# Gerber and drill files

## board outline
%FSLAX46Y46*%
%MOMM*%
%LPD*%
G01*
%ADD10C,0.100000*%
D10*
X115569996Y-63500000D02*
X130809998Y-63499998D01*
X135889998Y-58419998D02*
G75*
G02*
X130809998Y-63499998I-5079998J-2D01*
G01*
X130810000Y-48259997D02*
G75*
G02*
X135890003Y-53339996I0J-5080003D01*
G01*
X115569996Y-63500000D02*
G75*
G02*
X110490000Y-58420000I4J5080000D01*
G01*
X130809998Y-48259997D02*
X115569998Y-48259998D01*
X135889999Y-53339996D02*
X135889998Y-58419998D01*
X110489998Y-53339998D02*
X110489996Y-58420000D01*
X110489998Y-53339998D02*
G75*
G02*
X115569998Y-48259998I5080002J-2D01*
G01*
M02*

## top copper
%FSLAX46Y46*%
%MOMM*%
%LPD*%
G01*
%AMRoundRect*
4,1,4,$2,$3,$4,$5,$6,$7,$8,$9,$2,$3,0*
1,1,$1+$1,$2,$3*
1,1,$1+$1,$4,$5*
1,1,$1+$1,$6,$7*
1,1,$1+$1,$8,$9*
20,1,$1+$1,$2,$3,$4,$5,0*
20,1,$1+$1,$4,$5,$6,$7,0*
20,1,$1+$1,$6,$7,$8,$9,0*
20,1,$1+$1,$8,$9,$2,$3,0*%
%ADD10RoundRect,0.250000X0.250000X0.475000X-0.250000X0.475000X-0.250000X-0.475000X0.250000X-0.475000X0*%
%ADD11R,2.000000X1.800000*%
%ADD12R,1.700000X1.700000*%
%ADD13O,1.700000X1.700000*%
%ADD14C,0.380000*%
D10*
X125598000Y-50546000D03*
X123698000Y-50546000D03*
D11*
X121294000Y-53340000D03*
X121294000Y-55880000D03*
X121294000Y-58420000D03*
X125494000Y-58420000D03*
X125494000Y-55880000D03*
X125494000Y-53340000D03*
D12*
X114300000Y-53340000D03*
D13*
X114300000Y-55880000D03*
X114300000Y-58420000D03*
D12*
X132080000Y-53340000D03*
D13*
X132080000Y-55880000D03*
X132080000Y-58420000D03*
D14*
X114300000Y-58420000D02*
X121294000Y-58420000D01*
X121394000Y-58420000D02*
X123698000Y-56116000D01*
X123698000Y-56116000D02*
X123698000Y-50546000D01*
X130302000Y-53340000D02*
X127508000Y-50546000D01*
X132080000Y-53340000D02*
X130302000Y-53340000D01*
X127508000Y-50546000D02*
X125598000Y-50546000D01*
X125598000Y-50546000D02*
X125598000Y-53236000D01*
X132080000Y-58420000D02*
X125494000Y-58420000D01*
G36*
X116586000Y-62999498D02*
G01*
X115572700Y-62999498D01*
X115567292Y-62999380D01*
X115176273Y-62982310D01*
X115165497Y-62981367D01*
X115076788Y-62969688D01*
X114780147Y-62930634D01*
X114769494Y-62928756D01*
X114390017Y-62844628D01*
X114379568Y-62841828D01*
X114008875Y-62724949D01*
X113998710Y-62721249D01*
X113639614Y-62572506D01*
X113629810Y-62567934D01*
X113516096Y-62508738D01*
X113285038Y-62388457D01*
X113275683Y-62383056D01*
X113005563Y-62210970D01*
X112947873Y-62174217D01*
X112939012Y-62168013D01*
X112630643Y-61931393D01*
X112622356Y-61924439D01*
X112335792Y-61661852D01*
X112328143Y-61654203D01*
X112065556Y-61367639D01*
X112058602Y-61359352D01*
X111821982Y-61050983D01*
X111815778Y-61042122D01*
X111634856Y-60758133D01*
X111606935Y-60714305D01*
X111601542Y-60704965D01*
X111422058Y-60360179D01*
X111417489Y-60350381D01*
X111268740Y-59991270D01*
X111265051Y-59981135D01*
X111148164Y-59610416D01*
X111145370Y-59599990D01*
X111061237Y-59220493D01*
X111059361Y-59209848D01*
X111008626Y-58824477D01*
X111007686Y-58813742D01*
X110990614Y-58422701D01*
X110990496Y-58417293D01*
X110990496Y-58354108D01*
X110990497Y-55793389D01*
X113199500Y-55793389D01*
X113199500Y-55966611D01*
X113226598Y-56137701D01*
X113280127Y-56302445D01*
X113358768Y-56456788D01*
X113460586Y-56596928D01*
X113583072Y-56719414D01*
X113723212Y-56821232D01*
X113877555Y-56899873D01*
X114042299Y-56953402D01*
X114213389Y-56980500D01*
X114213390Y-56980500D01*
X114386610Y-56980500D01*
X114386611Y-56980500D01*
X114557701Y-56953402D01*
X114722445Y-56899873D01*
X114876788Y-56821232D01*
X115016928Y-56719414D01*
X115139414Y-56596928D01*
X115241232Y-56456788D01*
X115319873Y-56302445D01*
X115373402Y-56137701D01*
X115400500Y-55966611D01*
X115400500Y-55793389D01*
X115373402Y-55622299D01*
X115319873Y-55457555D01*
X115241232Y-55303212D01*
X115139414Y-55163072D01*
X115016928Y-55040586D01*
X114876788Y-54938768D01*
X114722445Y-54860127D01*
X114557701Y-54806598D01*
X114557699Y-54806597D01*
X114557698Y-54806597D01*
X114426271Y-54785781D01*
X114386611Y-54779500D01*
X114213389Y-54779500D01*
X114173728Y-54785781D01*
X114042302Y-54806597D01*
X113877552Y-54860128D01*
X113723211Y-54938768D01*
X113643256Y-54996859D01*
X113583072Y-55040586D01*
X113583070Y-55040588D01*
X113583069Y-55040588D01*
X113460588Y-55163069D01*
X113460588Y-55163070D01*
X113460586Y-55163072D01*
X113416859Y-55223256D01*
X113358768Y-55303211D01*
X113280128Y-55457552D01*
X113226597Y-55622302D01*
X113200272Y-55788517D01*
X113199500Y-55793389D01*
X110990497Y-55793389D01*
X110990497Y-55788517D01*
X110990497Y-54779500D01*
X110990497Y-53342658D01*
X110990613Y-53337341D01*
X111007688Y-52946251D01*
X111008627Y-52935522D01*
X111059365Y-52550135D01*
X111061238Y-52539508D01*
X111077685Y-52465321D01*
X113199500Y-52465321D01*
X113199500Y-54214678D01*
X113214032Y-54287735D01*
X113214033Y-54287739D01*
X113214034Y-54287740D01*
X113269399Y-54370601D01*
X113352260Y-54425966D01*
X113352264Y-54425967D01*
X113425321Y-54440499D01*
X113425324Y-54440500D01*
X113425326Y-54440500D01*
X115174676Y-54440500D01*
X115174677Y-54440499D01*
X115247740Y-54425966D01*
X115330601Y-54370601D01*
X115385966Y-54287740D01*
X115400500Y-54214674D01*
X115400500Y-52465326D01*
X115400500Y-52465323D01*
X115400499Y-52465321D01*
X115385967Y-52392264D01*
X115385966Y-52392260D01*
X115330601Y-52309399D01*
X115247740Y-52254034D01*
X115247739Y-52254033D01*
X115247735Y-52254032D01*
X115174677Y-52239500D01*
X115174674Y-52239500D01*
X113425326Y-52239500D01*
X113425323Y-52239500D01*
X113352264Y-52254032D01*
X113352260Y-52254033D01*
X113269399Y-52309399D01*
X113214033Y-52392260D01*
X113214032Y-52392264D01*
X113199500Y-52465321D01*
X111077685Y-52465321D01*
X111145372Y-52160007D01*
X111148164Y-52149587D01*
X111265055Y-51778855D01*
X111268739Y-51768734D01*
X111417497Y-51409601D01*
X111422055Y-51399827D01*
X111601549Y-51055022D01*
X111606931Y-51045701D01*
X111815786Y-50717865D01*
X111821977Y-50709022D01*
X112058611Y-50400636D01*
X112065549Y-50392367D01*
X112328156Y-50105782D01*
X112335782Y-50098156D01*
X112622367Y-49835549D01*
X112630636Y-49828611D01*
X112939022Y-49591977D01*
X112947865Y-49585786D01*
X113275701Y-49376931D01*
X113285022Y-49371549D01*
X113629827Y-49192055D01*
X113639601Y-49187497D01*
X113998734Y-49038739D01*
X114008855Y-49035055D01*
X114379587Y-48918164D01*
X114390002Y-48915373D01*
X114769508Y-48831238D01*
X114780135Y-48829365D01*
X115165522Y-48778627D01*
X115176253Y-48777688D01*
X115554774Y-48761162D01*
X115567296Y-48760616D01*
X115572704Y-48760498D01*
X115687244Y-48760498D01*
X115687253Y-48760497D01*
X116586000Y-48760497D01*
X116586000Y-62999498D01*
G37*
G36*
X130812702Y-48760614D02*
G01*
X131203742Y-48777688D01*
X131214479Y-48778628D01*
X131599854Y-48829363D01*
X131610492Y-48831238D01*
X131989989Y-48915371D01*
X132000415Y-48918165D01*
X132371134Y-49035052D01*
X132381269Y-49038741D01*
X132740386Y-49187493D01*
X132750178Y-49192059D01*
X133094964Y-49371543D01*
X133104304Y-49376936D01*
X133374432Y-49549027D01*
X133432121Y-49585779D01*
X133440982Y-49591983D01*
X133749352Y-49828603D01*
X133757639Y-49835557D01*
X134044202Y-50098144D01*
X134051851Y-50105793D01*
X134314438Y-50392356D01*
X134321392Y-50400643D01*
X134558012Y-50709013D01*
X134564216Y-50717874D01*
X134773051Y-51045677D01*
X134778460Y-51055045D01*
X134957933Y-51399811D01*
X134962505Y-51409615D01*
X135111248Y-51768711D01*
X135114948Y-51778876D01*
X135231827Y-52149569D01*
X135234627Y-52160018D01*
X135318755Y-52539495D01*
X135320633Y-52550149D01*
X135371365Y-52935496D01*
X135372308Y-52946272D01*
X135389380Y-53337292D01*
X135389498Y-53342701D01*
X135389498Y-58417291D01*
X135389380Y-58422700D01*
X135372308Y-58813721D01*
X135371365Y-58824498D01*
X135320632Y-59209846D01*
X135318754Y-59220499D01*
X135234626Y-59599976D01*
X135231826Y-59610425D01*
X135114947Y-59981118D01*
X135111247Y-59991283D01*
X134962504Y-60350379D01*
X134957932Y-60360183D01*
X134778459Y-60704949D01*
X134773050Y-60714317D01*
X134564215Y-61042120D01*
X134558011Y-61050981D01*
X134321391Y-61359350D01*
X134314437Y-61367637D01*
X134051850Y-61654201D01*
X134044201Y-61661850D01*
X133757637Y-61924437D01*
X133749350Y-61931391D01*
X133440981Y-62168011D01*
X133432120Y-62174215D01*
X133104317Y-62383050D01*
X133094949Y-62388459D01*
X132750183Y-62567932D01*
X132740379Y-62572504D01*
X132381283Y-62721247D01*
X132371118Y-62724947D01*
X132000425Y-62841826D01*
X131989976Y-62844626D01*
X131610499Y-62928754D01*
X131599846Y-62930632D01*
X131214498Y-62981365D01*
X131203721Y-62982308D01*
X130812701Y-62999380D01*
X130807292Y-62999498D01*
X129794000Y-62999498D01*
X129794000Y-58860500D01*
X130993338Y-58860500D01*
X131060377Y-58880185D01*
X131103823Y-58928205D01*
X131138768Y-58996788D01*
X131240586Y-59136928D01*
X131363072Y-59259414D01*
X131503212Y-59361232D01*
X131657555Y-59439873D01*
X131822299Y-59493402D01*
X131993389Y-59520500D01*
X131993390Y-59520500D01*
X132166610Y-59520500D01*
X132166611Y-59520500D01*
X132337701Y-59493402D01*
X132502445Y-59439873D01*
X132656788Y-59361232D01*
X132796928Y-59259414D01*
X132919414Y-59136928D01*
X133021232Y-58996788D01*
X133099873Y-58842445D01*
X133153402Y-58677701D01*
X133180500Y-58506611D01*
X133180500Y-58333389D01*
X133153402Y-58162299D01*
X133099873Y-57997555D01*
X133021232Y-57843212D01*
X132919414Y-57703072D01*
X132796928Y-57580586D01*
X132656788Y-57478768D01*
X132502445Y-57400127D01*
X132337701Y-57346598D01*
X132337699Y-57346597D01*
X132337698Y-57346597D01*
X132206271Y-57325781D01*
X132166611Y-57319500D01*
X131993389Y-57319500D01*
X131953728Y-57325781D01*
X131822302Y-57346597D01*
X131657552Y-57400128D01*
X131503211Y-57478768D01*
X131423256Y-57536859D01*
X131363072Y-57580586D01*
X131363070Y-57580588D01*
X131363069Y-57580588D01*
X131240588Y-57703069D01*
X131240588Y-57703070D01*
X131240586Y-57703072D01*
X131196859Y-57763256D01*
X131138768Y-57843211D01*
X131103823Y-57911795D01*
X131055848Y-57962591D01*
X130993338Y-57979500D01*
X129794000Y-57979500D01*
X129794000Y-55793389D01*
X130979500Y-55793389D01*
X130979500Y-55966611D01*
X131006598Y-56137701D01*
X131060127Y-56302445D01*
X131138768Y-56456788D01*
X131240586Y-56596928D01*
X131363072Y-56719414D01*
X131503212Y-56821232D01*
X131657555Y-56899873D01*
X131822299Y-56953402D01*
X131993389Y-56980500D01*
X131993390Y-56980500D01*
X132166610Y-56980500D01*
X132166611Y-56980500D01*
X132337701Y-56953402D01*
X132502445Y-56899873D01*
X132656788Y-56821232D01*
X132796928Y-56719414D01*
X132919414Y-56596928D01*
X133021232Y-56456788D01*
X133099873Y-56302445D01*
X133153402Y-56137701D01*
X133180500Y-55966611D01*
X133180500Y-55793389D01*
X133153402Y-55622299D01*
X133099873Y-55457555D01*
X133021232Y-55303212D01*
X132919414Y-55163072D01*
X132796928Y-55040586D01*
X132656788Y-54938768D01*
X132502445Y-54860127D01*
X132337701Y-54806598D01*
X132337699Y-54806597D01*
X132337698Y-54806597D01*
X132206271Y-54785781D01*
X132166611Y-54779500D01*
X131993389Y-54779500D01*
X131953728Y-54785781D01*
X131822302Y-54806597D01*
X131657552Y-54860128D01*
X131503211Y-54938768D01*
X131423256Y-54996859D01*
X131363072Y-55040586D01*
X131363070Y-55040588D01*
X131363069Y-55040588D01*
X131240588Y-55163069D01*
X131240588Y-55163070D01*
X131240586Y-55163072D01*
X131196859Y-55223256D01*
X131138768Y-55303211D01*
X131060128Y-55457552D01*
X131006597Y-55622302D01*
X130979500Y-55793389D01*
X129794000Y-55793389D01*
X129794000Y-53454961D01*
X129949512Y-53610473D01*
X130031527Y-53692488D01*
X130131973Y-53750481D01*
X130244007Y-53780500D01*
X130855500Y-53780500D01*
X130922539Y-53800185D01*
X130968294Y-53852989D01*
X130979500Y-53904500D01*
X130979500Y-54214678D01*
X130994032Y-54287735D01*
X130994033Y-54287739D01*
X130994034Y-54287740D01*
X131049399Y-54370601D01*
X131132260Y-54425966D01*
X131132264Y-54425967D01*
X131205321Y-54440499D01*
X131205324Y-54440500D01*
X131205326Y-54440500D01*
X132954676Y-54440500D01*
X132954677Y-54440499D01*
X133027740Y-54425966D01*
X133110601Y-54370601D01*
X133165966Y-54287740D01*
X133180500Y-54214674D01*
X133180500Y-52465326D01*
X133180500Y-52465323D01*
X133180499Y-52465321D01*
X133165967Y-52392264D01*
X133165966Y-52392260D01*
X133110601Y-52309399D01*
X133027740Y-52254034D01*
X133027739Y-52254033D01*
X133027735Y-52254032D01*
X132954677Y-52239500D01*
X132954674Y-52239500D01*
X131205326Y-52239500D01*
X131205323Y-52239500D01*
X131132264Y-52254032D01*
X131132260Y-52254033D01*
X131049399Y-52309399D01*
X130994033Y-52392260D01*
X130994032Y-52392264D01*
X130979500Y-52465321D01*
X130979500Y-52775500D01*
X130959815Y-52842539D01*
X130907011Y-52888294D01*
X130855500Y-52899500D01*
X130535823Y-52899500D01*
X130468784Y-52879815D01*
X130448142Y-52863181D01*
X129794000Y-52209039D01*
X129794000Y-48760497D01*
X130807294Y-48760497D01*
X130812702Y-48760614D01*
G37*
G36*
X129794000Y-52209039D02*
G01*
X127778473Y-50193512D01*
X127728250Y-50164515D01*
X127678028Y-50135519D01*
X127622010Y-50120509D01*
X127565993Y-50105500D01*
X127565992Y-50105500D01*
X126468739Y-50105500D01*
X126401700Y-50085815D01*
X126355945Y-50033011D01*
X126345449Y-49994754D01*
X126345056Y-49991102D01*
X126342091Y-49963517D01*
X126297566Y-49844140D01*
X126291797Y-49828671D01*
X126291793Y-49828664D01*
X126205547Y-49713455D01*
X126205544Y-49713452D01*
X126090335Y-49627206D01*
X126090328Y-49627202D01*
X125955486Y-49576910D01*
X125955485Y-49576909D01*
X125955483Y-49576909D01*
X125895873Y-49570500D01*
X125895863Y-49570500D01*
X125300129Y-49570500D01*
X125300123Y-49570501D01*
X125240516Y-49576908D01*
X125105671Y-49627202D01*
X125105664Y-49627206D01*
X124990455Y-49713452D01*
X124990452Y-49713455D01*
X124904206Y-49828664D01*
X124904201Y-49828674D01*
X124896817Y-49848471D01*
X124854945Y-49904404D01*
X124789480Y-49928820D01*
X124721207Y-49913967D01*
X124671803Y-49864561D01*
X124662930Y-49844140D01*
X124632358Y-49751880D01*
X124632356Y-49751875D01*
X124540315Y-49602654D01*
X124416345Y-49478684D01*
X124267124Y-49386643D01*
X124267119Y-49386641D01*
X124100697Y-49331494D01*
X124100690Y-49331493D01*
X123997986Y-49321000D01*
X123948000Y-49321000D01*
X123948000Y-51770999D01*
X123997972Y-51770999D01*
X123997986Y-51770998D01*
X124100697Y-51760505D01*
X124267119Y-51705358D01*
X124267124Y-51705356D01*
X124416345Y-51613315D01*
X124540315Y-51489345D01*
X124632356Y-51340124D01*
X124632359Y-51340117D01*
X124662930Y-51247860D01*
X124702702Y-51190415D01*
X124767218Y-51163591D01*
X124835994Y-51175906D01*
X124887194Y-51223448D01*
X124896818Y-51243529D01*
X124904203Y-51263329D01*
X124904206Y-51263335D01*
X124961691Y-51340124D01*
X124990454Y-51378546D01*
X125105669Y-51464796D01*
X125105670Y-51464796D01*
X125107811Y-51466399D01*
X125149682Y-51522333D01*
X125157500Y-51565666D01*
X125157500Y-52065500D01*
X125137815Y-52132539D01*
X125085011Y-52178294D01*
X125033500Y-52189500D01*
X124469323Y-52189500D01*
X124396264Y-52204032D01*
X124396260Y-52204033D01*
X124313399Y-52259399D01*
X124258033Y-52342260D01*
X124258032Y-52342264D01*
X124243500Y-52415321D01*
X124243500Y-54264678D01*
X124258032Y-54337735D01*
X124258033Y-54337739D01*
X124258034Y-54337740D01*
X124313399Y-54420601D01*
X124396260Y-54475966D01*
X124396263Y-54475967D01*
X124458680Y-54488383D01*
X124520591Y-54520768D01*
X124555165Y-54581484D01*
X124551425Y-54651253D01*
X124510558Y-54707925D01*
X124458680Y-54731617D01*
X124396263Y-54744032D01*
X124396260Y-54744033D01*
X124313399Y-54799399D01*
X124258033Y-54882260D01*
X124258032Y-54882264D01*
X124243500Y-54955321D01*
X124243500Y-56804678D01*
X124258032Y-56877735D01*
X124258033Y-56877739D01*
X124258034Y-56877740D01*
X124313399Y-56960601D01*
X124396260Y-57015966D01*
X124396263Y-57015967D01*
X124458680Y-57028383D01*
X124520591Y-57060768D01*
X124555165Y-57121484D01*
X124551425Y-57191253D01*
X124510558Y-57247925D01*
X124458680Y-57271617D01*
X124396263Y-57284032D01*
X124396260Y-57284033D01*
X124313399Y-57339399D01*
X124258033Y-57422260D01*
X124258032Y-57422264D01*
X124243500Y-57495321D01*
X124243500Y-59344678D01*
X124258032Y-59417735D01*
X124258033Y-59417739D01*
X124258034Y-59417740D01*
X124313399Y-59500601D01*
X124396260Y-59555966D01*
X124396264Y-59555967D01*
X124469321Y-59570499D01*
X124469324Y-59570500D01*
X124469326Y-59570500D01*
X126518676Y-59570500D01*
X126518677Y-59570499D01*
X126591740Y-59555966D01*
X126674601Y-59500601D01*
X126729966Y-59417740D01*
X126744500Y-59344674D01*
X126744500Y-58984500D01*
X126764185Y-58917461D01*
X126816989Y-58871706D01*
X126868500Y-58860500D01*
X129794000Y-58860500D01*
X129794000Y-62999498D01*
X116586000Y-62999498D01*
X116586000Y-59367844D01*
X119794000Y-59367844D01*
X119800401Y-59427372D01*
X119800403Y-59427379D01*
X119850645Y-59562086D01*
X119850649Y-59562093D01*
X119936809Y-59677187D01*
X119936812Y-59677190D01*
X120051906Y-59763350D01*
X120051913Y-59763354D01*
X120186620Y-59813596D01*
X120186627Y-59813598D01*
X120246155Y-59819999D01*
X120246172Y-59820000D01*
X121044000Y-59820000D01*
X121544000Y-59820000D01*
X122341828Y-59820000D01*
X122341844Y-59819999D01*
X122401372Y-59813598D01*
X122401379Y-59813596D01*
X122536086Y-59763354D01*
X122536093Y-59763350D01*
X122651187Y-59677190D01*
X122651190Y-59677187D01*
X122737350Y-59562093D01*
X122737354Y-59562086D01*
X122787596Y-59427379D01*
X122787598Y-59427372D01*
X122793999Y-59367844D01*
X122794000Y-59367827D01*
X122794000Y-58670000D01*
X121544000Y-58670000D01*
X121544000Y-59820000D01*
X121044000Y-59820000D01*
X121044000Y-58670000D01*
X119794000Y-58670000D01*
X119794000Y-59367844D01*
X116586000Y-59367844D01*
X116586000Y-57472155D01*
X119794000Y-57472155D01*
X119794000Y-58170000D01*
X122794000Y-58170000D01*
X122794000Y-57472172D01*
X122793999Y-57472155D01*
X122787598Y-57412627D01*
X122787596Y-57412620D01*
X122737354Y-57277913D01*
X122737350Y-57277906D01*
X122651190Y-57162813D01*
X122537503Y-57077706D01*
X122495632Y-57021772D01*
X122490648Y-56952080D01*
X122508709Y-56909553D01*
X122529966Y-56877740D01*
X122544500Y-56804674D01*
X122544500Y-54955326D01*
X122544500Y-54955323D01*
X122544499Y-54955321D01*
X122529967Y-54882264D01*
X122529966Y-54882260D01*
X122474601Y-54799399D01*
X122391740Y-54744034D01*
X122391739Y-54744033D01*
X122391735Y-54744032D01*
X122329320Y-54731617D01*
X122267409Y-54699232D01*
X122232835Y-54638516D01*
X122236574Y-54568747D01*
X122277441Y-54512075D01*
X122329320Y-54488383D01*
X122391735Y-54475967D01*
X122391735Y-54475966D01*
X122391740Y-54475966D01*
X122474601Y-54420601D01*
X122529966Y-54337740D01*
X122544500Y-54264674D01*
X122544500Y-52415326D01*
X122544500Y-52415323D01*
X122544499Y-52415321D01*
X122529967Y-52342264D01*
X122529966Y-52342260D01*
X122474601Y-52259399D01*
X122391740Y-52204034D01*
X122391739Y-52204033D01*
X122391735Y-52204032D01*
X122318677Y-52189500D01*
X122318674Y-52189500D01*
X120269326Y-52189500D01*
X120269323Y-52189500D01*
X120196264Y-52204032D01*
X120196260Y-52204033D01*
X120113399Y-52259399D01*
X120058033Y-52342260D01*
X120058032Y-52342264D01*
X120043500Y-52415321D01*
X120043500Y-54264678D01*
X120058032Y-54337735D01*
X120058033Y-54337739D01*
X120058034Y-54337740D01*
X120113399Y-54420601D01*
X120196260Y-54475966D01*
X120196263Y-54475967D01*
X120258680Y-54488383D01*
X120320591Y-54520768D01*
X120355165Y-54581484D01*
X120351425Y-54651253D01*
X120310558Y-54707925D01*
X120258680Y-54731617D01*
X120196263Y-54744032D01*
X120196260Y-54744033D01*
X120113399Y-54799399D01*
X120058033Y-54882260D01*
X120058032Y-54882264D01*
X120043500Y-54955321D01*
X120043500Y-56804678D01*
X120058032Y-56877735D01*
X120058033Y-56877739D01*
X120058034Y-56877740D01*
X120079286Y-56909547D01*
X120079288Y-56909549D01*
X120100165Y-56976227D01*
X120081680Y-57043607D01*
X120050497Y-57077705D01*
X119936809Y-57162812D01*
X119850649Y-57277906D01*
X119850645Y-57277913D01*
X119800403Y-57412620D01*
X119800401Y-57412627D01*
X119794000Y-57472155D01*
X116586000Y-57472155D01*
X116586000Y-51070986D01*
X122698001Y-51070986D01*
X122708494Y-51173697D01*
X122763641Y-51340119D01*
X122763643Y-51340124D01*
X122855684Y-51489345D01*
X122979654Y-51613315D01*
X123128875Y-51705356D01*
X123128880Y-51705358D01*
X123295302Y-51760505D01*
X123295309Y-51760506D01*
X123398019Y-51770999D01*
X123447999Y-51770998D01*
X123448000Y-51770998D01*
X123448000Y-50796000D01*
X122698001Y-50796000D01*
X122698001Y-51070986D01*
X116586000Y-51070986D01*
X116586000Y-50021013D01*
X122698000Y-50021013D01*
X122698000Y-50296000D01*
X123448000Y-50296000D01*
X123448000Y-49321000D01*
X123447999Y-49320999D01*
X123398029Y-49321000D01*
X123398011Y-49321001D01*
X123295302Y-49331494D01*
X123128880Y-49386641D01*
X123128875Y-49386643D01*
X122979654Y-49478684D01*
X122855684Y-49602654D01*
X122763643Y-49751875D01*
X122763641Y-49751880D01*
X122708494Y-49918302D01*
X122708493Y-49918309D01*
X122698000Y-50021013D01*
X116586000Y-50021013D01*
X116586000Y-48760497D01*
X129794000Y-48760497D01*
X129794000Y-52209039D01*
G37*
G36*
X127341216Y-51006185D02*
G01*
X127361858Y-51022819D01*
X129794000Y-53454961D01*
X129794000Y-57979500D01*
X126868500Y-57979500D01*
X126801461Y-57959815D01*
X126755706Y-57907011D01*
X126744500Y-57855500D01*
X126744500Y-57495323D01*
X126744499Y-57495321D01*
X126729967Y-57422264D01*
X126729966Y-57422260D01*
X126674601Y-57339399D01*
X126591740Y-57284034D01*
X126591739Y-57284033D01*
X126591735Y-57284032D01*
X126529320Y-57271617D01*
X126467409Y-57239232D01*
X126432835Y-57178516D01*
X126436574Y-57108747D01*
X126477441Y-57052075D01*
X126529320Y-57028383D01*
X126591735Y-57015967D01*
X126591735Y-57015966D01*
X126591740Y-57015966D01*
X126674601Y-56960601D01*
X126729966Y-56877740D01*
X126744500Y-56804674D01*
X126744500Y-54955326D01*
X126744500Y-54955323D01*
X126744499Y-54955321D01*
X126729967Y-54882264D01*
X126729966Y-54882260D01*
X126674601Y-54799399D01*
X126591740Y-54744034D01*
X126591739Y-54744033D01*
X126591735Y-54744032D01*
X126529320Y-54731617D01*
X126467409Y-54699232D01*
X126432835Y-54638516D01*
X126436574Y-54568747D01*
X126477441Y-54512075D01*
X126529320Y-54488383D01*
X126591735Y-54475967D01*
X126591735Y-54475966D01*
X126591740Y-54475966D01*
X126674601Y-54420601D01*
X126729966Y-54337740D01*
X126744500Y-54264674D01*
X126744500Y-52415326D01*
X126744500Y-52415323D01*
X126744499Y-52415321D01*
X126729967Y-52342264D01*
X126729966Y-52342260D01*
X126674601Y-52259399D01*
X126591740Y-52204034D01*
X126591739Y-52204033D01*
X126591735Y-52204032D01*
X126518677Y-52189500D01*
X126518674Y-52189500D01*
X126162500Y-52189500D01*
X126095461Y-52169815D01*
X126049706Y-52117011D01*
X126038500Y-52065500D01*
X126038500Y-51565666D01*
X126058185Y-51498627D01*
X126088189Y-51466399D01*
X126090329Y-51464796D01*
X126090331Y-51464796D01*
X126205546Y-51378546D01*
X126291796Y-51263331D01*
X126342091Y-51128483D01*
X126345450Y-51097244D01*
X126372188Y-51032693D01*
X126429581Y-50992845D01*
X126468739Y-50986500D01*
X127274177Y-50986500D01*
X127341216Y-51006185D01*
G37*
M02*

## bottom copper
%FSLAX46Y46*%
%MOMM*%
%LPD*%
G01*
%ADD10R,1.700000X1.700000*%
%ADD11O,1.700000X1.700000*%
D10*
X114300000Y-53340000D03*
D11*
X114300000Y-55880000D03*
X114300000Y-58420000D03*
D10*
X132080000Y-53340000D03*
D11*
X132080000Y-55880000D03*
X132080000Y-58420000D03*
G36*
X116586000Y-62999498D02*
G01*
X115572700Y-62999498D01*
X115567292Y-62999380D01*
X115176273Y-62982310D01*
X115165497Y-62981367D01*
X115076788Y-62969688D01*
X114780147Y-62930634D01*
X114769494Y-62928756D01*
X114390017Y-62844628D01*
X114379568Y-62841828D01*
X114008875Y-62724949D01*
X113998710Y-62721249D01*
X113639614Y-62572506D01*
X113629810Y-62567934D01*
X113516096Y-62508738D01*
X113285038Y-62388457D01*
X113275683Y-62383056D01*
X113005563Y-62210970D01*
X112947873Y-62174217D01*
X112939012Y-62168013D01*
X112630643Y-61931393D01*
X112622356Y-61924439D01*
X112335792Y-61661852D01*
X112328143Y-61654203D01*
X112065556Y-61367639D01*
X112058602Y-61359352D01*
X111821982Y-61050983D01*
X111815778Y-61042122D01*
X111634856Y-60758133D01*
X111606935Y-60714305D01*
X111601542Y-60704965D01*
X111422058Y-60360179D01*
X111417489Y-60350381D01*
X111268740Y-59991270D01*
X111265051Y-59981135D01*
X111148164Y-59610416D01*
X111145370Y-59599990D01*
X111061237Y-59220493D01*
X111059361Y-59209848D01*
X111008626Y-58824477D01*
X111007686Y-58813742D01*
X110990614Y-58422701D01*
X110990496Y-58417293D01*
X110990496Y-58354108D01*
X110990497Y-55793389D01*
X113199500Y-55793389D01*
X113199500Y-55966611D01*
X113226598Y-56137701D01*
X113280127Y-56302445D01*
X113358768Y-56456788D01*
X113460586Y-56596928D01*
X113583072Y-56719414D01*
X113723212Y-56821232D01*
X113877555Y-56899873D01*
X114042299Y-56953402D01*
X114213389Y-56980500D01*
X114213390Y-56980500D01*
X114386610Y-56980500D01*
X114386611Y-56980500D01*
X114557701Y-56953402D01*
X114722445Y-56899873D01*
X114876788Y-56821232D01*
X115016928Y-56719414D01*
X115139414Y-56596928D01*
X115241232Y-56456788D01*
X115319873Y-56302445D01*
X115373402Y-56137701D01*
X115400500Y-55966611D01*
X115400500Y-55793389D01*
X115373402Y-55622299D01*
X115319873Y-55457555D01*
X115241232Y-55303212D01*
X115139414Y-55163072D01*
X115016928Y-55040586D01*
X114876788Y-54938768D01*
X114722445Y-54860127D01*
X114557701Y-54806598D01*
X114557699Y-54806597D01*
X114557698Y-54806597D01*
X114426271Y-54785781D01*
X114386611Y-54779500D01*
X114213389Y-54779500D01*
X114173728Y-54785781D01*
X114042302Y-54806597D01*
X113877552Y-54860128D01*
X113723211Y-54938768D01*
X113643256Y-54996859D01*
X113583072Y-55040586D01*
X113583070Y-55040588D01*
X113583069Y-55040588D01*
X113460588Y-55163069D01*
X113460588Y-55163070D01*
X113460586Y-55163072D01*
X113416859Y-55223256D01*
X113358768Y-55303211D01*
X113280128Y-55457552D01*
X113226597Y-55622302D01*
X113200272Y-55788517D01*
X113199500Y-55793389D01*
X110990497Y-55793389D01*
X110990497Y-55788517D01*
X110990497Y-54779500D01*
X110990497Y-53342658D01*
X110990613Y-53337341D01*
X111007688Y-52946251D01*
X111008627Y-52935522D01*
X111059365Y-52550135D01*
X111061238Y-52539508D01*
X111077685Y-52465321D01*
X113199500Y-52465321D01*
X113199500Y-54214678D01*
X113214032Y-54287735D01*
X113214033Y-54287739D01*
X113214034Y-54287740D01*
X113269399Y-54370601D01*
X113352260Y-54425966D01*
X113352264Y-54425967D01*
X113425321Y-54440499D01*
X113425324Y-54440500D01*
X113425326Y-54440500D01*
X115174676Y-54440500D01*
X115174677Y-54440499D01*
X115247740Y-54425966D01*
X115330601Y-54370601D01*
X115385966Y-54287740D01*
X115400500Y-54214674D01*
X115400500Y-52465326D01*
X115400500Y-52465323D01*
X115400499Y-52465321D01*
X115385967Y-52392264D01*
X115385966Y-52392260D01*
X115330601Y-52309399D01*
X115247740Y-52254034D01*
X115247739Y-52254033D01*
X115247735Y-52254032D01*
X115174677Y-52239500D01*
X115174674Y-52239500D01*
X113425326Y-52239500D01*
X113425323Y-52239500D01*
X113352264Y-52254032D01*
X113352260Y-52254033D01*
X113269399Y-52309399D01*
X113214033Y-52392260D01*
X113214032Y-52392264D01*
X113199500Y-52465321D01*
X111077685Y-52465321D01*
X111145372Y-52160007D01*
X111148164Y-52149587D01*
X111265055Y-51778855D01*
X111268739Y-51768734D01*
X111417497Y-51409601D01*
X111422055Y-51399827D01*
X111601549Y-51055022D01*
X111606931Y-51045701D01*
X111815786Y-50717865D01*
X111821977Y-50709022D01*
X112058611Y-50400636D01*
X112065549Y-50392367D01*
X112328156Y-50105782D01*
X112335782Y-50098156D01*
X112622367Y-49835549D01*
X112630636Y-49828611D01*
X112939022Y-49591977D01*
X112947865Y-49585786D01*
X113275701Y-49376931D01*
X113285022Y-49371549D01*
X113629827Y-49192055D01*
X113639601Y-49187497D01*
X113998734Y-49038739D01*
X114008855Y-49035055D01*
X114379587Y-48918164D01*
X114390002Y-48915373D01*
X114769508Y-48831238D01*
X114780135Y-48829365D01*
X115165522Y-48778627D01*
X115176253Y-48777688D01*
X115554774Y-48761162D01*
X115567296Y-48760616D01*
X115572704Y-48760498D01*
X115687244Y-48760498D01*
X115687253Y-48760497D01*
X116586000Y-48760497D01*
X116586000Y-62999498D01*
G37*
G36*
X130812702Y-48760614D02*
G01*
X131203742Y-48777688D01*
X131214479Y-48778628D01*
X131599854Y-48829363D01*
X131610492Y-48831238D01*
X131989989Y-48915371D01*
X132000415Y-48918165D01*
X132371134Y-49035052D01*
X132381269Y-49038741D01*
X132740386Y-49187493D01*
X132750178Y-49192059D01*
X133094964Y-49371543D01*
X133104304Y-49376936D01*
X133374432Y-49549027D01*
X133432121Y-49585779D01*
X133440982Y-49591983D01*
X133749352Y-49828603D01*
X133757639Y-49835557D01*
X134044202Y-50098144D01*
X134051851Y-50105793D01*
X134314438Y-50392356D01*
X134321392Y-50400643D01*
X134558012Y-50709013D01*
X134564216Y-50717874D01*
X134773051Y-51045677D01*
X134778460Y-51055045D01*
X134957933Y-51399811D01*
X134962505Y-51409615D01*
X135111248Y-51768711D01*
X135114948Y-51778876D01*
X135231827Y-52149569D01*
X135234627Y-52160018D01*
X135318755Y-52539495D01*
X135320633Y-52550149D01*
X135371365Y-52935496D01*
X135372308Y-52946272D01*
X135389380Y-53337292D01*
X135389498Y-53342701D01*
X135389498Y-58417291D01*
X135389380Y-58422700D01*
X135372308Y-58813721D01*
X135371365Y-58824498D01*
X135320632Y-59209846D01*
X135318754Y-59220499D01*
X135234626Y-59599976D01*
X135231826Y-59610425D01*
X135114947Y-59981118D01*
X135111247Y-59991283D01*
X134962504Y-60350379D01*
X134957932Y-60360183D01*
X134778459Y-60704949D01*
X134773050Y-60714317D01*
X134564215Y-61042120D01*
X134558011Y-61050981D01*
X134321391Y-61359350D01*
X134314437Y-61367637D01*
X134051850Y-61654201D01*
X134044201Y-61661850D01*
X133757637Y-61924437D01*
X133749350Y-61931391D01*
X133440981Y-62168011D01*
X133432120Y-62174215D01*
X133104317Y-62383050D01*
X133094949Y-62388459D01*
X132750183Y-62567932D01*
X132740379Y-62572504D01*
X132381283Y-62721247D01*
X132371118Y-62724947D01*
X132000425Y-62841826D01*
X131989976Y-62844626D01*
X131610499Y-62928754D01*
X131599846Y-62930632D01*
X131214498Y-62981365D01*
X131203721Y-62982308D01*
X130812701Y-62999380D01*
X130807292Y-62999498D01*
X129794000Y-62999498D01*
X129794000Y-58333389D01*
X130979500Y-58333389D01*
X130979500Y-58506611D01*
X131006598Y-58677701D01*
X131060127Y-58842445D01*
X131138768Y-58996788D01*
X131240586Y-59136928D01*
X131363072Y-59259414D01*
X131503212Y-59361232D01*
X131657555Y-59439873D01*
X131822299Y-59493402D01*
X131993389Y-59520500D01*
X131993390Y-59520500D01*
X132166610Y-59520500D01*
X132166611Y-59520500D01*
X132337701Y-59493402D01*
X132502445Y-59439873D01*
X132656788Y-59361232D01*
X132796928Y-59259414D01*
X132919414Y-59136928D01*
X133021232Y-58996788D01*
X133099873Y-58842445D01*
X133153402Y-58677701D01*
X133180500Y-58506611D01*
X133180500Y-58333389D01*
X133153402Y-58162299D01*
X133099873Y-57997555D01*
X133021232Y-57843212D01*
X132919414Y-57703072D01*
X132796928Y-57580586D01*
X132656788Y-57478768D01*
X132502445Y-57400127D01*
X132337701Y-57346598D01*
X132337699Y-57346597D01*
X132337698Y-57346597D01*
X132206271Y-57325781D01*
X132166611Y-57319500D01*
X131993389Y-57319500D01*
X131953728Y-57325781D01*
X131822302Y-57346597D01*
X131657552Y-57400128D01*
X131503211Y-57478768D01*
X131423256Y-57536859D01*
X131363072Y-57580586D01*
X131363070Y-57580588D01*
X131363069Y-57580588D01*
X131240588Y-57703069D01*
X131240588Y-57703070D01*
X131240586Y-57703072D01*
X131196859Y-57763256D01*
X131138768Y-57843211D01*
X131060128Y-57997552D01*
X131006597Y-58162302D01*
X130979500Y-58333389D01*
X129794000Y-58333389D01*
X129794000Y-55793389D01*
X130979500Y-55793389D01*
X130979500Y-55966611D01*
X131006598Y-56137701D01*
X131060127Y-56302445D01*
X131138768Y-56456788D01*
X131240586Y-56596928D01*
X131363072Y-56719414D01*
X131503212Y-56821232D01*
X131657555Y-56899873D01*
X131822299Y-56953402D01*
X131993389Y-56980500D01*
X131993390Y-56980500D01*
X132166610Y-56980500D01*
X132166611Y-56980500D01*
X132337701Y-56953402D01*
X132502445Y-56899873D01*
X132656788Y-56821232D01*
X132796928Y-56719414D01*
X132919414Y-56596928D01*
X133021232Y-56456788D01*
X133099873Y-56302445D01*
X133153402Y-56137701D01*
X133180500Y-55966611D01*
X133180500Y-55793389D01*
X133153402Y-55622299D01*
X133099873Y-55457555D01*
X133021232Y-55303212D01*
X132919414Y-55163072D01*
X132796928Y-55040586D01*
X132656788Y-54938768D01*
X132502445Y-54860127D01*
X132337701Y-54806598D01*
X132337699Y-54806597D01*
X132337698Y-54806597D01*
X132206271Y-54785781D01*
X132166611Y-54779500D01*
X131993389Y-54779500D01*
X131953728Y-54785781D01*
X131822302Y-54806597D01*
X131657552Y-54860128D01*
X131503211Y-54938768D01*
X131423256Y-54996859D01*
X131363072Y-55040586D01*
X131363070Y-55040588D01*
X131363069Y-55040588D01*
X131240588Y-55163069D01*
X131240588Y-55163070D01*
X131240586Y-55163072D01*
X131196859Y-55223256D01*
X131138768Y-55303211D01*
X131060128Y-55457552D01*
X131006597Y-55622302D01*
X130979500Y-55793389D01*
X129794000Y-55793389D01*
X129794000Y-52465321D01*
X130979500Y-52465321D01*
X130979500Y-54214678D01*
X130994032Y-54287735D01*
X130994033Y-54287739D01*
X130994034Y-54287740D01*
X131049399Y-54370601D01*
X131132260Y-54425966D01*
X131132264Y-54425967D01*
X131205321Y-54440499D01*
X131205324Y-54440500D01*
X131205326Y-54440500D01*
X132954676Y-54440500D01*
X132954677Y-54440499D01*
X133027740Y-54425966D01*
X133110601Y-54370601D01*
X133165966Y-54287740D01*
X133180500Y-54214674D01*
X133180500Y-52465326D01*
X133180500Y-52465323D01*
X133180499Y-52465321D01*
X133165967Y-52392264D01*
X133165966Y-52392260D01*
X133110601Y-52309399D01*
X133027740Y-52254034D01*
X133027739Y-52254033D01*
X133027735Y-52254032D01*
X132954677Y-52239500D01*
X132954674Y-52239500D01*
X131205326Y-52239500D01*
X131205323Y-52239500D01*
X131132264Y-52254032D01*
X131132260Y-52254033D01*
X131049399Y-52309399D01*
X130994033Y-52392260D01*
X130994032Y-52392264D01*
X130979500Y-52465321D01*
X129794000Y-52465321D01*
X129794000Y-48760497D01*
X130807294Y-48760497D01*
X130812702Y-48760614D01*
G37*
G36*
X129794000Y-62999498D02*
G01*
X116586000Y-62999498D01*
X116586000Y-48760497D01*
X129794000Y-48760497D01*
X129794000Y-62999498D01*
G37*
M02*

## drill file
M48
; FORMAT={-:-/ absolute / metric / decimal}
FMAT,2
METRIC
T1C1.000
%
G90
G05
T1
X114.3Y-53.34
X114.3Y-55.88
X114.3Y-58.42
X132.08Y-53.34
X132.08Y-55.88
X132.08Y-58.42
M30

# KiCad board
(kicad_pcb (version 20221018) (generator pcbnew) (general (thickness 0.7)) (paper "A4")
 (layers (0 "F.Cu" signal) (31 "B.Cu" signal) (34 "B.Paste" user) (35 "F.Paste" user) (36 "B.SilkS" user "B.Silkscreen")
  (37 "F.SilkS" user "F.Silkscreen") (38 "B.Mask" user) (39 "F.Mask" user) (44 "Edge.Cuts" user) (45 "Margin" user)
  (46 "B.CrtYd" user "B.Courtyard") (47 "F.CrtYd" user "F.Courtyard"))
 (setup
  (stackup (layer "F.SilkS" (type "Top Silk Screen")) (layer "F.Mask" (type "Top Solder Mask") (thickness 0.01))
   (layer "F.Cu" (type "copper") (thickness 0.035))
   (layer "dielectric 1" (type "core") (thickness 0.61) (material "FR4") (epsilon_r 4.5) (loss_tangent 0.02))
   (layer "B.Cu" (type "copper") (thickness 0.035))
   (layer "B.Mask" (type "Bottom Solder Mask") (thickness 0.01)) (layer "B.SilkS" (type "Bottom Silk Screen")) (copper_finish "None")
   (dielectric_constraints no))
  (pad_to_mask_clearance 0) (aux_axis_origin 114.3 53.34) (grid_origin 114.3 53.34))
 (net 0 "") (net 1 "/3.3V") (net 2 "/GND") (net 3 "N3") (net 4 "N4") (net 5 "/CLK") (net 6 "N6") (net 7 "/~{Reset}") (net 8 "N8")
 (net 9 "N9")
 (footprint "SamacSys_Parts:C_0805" (layer "F.Cu") (at 124.664 50.546 90)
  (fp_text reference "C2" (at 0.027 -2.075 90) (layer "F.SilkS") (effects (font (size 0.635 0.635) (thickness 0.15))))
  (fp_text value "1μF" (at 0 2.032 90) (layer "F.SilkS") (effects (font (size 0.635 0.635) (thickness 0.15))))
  (pad "1" smd roundrect (at 0 0.934 180) (size 1 1.45) (layers "F.Cu" "F.Paste" "F.Mask") (roundrect_rratio 0.25) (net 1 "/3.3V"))
  (pad "2" smd roundrect (at 0 -0.966 180) (size 1 1.45) (layers "F.Cu" "F.Paste" "F.Mask") (roundrect_rratio 0.25) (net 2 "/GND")))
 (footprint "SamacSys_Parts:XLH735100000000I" (layer "F.Cu") (at 123.394 55.88 -90)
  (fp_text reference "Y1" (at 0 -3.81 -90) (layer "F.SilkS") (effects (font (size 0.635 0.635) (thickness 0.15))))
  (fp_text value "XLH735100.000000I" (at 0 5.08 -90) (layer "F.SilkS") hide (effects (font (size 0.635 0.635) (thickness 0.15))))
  (pad "1" smd rect (at -2.54 2.1 270) (size 1.8 2) (layers "F.Cu" "F.Paste" "F.Mask") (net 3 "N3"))
  (pad "2" smd rect (at 0 2.1 270) (size 1.8 2) (layers "F.Cu" "F.Paste" "F.Mask") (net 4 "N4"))
  (pad "3" smd rect (at 2.54 2.1 270) (size 1.8 2) (layers "F.Cu" "F.Paste" "F.Mask") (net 2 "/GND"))
  (pad "4" smd rect (at 2.54 -2.1 270) (size 1.8 2) (layers "F.Cu" "F.Paste" "F.Mask") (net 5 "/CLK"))
  (pad "5" smd rect (at 0 -2.1 270) (size 1.8 2) (layers "F.Cu" "F.Paste" "F.Mask") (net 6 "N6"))
  (pad "6" smd rect (at -2.54 -2.1 270) (size 1.8 2) (layers "F.Cu" "F.Paste" "F.Mask") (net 1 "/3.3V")))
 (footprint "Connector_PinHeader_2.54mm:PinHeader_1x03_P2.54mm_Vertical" (layer "B.Cu") (at 114.3 53.34 180)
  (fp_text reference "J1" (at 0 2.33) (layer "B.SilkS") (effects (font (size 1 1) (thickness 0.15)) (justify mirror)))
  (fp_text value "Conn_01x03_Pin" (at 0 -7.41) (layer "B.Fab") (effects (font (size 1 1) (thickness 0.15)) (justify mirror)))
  (pad "1" thru_hole rect (at 0 0 180) (size 1.7 1.7) (drill 1) (layers "*.Cu" "*.Mask") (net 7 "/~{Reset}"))
  (pad "2" thru_hole oval (at 0 -2.54 180) (size 1.7 1.7) (drill 1) (layers "*.Cu" "*.Mask") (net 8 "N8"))
  (pad "3" thru_hole oval (at 0 -5.08 180) (size 1.7 1.7) (drill 1) (layers "*.Cu" "*.Mask") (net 2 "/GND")))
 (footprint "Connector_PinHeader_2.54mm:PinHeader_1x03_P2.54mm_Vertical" (layer "B.Cu") (at 132.08 53.34 180)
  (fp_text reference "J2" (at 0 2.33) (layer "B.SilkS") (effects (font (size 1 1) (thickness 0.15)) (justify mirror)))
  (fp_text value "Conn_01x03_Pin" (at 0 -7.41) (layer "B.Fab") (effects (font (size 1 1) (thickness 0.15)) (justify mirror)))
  (pad "1" thru_hole rect (at 0 0 180) (size 1.7 1.7) (drill 1) (layers "*.Cu" "*.Mask") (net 1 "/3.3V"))
  (pad "2" thru_hole oval (at 0 -2.54 180) (size 1.7 1.7) (drill 1) (layers "*.Cu" "*.Mask") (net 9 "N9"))
  (pad "3" thru_hole oval (at 0 -5.08 180) (size 1.7 1.7) (drill 1) (layers "*.Cu" "*.Mask") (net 5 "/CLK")))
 (gr_line (start 115.569996 63.5) (end 130.809998 63.499998) (stroke (width 0.1) (type default)) (layer "Edge.Cuts"))
 (gr_arc (start 135.889998 58.419998) (mid 134.4021 62.0121) (end 130.809998 63.499998) (stroke (width 0.1) (type default))
  (layer "Edge.Cuts"))
 (gr_arc (start 130.81 48.259997) (mid 134.402101 49.747895) (end 135.889999 53.339996) (stroke (width 0.1) (type default))
  (layer "Edge.Cuts"))
 (gr_arc (start 115.569996 63.5) (mid 111.977894 62.012102) (end 110.489996 58.42) (stroke (width 0.1) (type default)) (layer "Edge.Cuts"))
 (gr_line (start 130.809998 48.259997) (end 115.569998 48.259998) (stroke (width 0.1) (type default)) (layer "Edge.Cuts"))
 (gr_line (start 135.889999 53.339996) (end 135.889998 58.419998) (stroke (width 0.1) (type default)) (layer "Edge.Cuts"))
 (gr_line (start 110.489998 53.339998) (end 110.489996 58.42) (stroke (width 0.1) (type default)) (layer "Edge.Cuts"))
 (gr_arc (start 110.489998 53.339998) (mid 111.977896 49.747896) (end 115.569998 48.259998) (stroke (width 0.1) (type default))
  (layer "Edge.Cuts"))
 (segment (start 114.3 58.42) (end 121.294 58.42) (width 0.38) (layer "F.Cu") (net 2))
 (segment (start 121.394 58.42) (end 123.698 56.116) (width 0.38) (layer "F.Cu") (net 2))
 (segment (start 123.698 56.116) (end 123.698 50.546) (width 0.38) (layer "F.Cu") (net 2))
 (segment (start 130.302 53.34) (end 127.508 50.546) (width 0.38) (layer "F.Cu") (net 1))
 (segment (start 132.08 53.34) (end 130.302 53.34) (width 0.38) (layer "F.Cu") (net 1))
 (segment (start 127.508 50.546) (end 125.598 50.546) (width 0.38) (layer "F.Cu") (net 1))
 (segment (start 125.598 50.546) (end 125.598 53.236) (width 0.38) (layer "F.Cu") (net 1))
 (segment (start 132.08 58.42) (end 125.494 58.42) (width 0.38) (layer "F.Cu") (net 5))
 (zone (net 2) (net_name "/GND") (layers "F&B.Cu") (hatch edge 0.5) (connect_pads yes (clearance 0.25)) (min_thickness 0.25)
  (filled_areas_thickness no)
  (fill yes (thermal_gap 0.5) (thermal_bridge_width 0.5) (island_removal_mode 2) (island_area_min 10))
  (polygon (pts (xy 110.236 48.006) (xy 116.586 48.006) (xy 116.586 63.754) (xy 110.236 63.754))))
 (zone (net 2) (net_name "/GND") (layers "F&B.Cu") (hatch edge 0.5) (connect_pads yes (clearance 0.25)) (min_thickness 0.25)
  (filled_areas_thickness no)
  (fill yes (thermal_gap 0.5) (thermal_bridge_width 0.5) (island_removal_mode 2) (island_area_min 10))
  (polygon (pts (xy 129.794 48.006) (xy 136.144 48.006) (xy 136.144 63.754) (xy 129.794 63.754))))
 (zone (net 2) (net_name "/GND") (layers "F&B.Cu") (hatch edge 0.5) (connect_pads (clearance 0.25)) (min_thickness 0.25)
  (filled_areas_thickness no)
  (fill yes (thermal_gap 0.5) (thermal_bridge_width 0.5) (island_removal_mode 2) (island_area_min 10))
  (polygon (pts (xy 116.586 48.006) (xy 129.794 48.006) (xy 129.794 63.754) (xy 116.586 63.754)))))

